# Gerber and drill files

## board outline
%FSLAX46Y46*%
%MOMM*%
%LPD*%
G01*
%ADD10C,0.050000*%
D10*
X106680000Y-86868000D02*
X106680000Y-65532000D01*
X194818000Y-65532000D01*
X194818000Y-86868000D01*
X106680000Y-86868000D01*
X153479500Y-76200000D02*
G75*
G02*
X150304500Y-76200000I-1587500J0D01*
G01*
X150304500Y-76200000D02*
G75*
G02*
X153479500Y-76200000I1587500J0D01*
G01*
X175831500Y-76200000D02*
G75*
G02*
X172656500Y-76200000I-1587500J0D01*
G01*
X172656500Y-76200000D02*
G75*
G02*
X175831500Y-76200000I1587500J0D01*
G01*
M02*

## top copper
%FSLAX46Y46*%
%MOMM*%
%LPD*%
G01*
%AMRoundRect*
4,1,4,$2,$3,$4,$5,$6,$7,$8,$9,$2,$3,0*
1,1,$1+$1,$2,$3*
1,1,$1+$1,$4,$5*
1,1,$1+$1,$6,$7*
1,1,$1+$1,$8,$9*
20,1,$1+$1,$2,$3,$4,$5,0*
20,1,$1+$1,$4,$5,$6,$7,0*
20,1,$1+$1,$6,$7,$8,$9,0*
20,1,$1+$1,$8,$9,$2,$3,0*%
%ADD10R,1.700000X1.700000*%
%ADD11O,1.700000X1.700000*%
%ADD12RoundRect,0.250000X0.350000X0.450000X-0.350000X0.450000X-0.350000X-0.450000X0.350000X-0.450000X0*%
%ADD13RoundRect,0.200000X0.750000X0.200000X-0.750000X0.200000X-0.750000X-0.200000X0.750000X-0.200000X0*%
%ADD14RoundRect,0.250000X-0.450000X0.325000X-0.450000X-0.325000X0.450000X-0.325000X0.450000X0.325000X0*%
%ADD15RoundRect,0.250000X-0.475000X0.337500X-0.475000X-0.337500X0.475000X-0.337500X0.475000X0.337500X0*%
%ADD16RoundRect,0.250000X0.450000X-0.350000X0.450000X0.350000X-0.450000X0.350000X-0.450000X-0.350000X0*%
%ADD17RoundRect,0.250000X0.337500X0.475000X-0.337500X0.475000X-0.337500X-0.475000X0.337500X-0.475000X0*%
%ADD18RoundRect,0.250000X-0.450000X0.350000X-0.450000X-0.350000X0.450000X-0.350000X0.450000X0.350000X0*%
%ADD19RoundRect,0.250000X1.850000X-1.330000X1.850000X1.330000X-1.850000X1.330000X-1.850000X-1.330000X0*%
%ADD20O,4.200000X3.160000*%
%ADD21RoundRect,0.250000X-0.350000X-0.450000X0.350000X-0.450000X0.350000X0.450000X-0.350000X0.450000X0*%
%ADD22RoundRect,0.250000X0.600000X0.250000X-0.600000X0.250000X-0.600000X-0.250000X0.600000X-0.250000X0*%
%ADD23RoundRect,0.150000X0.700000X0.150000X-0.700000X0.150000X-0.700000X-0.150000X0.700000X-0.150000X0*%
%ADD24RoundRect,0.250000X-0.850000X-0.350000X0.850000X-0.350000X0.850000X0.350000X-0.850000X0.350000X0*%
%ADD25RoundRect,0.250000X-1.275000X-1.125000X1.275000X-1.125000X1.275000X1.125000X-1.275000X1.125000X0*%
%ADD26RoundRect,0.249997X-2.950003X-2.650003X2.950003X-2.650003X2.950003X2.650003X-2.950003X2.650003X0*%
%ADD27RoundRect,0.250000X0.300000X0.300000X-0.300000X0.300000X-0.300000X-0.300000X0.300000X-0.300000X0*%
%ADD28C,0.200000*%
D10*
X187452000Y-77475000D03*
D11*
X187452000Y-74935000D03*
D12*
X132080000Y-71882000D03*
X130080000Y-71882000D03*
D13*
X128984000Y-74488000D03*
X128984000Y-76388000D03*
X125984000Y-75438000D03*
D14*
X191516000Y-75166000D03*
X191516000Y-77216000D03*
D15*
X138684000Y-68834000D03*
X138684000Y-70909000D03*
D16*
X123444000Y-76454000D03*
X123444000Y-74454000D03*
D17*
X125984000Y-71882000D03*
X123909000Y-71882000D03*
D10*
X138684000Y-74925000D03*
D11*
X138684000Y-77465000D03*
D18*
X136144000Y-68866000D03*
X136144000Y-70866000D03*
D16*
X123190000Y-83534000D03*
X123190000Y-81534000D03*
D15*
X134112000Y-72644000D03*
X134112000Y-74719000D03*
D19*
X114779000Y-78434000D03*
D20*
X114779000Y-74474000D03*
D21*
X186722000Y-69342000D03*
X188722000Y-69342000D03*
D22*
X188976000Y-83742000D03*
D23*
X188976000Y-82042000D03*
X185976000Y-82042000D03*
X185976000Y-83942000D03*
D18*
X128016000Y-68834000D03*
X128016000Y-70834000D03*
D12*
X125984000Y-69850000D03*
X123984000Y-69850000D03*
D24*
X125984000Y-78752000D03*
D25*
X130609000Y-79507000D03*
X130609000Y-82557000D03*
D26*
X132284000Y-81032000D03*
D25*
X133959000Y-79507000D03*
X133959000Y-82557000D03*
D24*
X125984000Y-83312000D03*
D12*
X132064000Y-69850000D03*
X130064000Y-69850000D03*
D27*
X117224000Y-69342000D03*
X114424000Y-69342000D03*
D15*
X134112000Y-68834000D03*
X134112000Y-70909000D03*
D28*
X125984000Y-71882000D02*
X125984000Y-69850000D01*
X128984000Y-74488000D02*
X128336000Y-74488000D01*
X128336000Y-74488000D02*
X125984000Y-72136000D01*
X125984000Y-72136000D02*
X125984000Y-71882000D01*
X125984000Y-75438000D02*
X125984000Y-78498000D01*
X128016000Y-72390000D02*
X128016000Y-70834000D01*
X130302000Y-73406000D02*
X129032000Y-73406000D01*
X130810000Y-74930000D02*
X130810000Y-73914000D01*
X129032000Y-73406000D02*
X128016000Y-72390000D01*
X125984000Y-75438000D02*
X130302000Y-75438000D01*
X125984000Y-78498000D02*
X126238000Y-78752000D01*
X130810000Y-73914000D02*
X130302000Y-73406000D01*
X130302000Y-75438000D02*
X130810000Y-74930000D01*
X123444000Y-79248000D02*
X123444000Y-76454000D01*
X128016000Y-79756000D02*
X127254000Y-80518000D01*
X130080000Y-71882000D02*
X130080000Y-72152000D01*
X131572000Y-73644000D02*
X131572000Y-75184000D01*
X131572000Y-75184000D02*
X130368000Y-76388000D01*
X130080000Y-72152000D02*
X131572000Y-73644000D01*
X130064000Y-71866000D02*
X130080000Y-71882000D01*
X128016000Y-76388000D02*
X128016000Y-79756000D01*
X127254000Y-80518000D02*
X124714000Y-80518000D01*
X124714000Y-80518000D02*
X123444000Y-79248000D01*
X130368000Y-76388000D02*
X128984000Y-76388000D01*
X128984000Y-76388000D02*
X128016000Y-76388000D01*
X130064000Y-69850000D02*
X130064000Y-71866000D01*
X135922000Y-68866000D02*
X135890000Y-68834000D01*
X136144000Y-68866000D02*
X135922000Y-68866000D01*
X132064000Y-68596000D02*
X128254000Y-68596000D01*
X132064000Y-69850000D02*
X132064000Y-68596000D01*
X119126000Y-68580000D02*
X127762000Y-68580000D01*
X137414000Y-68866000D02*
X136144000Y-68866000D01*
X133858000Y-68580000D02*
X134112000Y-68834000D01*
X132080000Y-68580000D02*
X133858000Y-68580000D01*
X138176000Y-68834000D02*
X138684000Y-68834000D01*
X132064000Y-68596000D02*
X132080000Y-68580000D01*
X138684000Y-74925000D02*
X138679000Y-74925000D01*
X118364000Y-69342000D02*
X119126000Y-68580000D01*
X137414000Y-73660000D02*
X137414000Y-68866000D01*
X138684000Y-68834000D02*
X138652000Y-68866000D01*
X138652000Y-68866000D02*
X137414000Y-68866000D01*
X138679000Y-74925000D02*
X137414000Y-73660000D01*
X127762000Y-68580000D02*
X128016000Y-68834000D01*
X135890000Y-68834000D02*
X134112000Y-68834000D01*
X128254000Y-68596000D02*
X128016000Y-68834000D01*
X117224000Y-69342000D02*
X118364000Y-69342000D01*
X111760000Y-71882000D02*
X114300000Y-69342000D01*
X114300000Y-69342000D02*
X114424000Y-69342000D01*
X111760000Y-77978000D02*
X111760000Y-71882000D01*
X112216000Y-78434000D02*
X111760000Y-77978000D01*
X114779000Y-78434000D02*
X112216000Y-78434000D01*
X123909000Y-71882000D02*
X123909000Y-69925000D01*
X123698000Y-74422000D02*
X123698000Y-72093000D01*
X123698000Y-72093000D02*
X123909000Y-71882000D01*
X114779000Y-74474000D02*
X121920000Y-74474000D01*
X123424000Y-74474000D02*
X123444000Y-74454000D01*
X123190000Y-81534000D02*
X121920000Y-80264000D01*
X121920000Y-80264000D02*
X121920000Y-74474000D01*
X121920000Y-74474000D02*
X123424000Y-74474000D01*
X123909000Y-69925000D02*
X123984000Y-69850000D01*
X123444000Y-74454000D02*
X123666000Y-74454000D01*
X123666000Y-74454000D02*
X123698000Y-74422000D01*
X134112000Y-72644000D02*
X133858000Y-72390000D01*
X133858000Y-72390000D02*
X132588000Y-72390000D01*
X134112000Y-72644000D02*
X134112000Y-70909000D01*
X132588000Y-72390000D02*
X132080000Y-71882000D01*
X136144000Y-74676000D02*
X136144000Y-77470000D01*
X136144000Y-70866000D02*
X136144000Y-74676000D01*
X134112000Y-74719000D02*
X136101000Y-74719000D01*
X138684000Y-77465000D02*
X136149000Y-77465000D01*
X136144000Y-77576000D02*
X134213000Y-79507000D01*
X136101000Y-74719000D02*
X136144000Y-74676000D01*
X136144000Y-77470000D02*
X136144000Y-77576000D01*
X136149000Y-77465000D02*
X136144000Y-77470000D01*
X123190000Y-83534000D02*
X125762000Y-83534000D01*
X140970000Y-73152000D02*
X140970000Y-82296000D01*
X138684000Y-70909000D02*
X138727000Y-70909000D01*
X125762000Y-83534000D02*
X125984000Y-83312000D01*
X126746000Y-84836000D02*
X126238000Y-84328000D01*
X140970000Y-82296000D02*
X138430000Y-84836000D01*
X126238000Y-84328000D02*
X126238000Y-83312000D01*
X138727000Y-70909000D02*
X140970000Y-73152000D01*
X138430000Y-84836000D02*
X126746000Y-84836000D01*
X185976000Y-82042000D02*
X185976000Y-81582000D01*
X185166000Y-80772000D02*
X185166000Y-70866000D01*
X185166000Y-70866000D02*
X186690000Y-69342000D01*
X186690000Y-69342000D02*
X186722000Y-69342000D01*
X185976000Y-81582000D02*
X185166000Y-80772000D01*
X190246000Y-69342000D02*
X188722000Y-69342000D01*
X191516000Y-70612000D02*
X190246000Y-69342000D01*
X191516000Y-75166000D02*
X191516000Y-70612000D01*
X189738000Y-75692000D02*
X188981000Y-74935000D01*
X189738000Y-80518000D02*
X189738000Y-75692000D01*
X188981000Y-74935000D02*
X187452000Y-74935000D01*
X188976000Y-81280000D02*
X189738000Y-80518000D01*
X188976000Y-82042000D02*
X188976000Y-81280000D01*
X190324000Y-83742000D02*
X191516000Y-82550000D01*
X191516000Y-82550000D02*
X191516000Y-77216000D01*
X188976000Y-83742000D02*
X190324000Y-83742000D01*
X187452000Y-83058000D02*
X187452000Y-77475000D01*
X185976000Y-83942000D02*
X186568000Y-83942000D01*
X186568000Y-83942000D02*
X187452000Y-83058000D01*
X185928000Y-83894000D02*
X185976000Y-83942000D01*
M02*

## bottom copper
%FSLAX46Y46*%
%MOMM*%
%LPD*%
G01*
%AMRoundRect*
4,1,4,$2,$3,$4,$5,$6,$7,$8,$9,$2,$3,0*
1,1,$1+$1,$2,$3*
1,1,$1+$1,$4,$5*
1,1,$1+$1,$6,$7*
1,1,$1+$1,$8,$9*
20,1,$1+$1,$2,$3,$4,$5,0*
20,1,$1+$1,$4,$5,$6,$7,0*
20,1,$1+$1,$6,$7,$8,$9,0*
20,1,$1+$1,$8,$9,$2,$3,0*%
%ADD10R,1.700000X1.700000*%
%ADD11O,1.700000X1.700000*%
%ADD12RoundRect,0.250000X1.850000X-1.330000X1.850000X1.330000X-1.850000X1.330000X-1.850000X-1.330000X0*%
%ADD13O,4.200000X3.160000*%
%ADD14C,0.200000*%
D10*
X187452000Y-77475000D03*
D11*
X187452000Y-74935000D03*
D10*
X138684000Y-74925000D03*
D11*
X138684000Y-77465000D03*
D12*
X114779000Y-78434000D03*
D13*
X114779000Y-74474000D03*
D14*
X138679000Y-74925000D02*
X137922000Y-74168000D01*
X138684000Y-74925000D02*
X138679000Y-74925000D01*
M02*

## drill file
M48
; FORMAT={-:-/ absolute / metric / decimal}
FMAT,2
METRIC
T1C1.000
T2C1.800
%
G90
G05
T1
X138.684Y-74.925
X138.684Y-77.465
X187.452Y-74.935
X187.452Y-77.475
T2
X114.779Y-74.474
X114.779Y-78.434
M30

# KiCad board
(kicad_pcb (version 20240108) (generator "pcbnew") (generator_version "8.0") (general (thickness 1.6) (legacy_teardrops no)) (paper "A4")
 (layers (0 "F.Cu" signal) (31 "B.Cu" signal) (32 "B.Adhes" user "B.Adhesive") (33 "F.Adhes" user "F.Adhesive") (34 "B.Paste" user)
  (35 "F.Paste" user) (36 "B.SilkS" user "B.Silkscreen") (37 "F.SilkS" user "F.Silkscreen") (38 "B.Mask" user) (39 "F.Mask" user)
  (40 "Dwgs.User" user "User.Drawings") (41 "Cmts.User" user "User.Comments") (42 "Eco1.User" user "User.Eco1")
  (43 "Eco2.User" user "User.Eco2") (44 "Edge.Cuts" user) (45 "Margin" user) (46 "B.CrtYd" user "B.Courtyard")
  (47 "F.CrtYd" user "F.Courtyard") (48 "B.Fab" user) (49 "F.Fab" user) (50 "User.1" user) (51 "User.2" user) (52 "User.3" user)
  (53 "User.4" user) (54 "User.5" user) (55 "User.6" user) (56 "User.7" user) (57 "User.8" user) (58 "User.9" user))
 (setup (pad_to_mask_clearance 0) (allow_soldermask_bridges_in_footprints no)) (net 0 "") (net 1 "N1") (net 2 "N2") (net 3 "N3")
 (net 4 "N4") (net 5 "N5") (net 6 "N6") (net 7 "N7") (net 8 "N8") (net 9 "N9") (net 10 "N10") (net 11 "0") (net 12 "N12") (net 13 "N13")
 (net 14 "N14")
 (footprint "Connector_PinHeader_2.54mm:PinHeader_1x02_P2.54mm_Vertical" (layer "F.Cu") (at 187.452 77.475 180)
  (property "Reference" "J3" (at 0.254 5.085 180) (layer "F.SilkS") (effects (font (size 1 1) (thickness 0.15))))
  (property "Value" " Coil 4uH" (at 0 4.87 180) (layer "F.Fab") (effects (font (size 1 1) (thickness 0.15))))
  (pad "1" thru_hole rect (at 0 0 180) (size 1.7 1.7) (drill 1) (layers "*.Cu" "*.Mask") (remove_unused_layers no) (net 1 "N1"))
  (pad "2" thru_hole oval (at 0 2.54 180) (size 1.7 1.7) (drill 1) (layers "*.Cu" "*.Mask") (remove_unused_layers no) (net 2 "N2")))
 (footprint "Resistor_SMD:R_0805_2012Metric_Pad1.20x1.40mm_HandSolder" (layer "F.Cu") (at 131.08 71.882 180)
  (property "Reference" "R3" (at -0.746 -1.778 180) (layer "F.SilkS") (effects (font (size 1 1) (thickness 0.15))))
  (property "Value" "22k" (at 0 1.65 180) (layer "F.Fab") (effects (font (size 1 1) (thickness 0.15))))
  (pad "1" smd roundrect (at -1 0 180) (size 1.2 1.4) (layers "F.Cu" "F.Paste" "F.Mask") (roundrect_rratio 0.208333) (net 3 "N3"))
  (pad "2" smd roundrect (at 1 0 180) (size 1.2 1.4) (layers "F.Cu" "F.Paste" "F.Mask") (roundrect_rratio 0.208333) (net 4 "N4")))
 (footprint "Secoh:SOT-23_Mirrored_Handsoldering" (layer "F.Cu") (at 127.484 75.438 180)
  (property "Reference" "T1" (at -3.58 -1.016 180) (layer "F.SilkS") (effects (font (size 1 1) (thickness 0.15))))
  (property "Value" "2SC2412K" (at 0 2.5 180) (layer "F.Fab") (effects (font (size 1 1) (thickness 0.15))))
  (pad "1" smd roundrect (at -1.5 0.95 180) (size 1.9 0.8) (layers "F.Cu" "F.Paste" "F.Mask") (roundrect_rratio 0.25) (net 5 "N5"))
  (pad "2" smd roundrect (at -1.5 -0.95 180) (size 1.9 0.8) (layers "F.Cu" "F.Paste" "F.Mask") (roundrect_rratio 0.25) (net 4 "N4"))
  (pad "3" smd roundrect (at 1.5 0 180) (size 1.9 0.8) (layers "F.Cu" "F.Paste" "F.Mask") (roundrect_rratio 0.25) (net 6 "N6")))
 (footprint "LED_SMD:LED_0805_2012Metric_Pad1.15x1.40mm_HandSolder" (layer "F.Cu") (at 191.516 76.191 -90)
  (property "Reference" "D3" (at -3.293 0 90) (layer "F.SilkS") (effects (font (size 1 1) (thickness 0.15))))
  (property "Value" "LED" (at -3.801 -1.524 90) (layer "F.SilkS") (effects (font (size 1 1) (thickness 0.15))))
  (pad "1" smd roundrect (at -1.025 0 270) (size 1.15 1.4) (layers "F.Cu" "F.Paste" "F.Mask") (roundrect_rratio 0.217391) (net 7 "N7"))
  (pad "2" smd roundrect (at 1.025 0 270) (size 1.15 1.4) (layers "F.Cu" "F.Paste" "F.Mask") (roundrect_rratio 0.217391) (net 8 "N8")))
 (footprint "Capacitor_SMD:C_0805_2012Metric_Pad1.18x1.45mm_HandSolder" (layer "F.Cu") (at 138.684 69.8715 -90)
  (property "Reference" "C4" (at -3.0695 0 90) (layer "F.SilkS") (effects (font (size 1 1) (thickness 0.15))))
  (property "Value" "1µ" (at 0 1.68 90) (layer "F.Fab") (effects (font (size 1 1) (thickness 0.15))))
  (pad "1" smd roundrect (at -1.0375 0 270) (size 1.175 1.45) (layers "F.Cu" "F.Paste" "F.Mask") (roundrect_rratio 0.212766) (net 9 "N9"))
  (pad "2" smd roundrect (at 1.0375 0 270) (size 1.175 1.45) (layers "F.Cu" "F.Paste" "F.Mask") (roundrect_rratio 0.212766) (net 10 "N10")))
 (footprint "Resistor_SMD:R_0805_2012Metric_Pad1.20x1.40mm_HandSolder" (layer "F.Cu") (at 123.444 75.454 90)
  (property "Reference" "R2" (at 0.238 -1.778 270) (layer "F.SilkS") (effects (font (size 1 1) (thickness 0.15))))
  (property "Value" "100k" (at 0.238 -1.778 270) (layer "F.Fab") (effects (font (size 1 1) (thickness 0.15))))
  (pad "1" smd roundrect (at -1 0 90) (size 1.2 1.4) (layers "F.Cu" "F.Paste" "F.Mask") (roundrect_rratio 0.208333) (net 4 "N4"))
  (pad "2" smd roundrect (at 1 0 90) (size 1.2 1.4) (layers "F.Cu" "F.Paste" "F.Mask") (roundrect_rratio 0.208333) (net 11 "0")))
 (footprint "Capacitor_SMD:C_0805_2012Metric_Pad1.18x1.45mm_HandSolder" (layer "F.Cu") (at 124.9465 71.882 180)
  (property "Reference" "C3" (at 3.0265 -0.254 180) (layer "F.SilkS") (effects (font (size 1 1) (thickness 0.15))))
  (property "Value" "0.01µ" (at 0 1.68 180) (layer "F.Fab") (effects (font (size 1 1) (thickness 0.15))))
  (pad "1" smd roundrect (at -1.0375 0 180) (size 1.175 1.45) (layers "F.Cu" "F.Paste" "F.Mask") (roundrect_rratio 0.212766) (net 5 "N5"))
  (pad "2" smd roundrect (at 1.0375 0 180) (size 1.175 1.45) (layers "F.Cu" "F.Paste" "F.Mask") (roundrect_rratio 0.212766) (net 11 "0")))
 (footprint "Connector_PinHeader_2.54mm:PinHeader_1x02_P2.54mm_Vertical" (layer "F.Cu") (at 138.684 74.925)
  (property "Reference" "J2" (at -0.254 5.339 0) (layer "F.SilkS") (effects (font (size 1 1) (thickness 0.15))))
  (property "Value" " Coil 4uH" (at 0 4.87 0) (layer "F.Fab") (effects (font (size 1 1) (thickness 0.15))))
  (pad "1" thru_hole rect (at 0 0) (size 1.7 1.7) (drill 1) (layers "*.Cu" "*.Mask") (remove_unused_layers no) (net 9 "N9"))
  (pad "2" thru_hole oval (at 0 2.54) (size 1.7 1.7) (drill 1) (layers "*.Cu" "*.Mask") (remove_unused_layers no) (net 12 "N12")))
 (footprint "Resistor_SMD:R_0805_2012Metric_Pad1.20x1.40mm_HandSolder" (layer "F.Cu") (at 136.144 69.866 -90)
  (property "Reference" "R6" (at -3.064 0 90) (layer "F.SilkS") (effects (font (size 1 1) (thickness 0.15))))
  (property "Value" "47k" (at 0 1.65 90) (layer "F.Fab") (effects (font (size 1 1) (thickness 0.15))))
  (pad "1" smd roundrect (at -1 0 270) (size 1.2 1.4) (layers "F.Cu" "F.Paste" "F.Mask") (roundrect_rratio 0.208333) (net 9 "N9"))
  (pad "2" smd roundrect (at 1 0 270) (size 1.2 1.4) (layers "F.Cu" "F.Paste" "F.Mask") (roundrect_rratio 0.208333) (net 12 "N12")))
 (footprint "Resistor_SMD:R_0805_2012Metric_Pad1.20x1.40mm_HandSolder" (layer "F.Cu") (at 123.19 82.534 90)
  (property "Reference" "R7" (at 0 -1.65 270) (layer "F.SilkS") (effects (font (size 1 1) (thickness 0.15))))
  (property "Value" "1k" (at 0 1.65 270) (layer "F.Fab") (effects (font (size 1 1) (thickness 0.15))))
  (pad "1" smd roundrect (at -1 0 90) (size 1.2 1.4) (layers "F.Cu" "F.Paste" "F.Mask") (roundrect_rratio 0.208333) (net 10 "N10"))
  (pad "2" smd roundrect (at 1 0 90) (size 1.2 1.4) (layers "F.Cu" "F.Paste" "F.Mask") (roundrect_rratio 0.208333) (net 11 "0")))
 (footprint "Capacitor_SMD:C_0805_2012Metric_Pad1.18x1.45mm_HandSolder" (layer "F.Cu") (at 134.112 73.6815 -90)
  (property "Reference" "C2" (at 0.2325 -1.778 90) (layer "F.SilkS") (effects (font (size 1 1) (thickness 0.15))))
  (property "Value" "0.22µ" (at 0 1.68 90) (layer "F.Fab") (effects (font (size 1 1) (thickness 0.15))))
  (pad "1" smd roundrect (at -1.0375 0 270) (size 1.175 1.45) (layers "F.Cu" "F.Paste" "F.Mask") (roundrect_rratio 0.212766) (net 3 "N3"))
  (pad "2" smd roundrect (at 1.0375 0 270) (size 1.175 1.45) (layers "F.Cu" "F.Paste" "F.Mask") (roundrect_rratio 0.212766) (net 12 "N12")))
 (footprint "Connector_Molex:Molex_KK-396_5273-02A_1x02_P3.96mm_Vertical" (layer "F.Cu") (at 114.779 78.434 90)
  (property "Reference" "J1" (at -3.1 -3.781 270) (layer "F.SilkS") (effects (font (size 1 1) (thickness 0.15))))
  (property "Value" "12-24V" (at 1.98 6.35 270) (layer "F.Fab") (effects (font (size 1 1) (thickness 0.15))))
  (pad "1" thru_hole roundrect (at 0 0 90) (size 3.16 4.2) (drill 1.8) (layers "*.Cu" "*.Mask") (remove_unused_layers no)
   (roundrect_rratio 0.079114) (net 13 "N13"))
  (pad "2" thru_hole oval (at 3.96 0 90) (size 3.16 4.2) (drill 1.8) (layers "*.Cu" "*.Mask") (remove_unused_layers no) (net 11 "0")))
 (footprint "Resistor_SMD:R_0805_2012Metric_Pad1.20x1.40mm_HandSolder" (layer "F.Cu") (at 187.722 69.342)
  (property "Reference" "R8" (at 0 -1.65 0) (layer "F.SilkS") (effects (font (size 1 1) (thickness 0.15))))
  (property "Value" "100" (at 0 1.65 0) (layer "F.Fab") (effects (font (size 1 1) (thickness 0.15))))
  (pad "1" smd roundrect (at -1 0) (size 1.2 1.4) (layers "F.Cu" "F.Paste" "F.Mask") (roundrect_rratio 0.208333) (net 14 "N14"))
  (pad "2" smd roundrect (at 1 0) (size 1.2 1.4) (layers "F.Cu" "F.Paste" "F.Mask") (roundrect_rratio 0.208333) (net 7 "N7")))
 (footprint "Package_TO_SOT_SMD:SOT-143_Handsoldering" (layer "F.Cu") (at 187.476 82.992 180)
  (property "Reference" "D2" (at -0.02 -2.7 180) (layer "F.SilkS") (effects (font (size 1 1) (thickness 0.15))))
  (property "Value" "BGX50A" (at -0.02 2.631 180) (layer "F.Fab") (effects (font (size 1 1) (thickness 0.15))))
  (pad "1" smd roundrect (at -1.5 -0.75 180) (size 1.7 1) (layers "F.Cu" "F.Paste" "F.Mask") (roundrect_rratio 0.25) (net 8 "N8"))
  (pad "2" smd roundrect (at -1.5 0.95 180) (size 1.7 0.6) (layers "F.Cu" "F.Paste" "F.Mask") (roundrect_rratio 0.25) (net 2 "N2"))
  (pad "3" smd roundrect (at 1.5 0.95 180) (size 1.7 0.6) (layers "F.Cu" "F.Paste" "F.Mask") (roundrect_rratio 0.25) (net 14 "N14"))
  (pad "4" smd roundrect (at 1.5 -0.95 180) (size 1.7 0.6) (layers "F.Cu" "F.Paste" "F.Mask") (roundrect_rratio 0.25) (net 1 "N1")))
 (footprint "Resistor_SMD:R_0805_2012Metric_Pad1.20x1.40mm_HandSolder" (layer "F.Cu") (at 128.016 69.834 -90)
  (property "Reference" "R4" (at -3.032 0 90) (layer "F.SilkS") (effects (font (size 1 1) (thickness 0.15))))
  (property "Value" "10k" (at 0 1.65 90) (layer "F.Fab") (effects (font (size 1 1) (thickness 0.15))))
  (pad "1" smd roundrect (at -1 0 270) (size 1.2 1.4) (layers "F.Cu" "F.Paste" "F.Mask") (roundrect_rratio 0.208333) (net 9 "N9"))
  (pad "2" smd roundrect (at 1 0 270) (size 1.2 1.4) (layers "F.Cu" "F.Paste" "F.Mask") (roundrect_rratio 0.208333) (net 6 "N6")))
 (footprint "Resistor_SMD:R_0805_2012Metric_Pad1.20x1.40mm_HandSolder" (layer "F.Cu") (at 124.984 69.85 180)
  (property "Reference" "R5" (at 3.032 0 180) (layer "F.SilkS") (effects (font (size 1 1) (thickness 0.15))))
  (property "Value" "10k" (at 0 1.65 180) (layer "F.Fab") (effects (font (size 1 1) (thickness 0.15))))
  (pad "1" smd roundrect (at -1 0 180) (size 1.2 1.4) (layers "F.Cu" "F.Paste" "F.Mask") (roundrect_rratio 0.208333) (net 5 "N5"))
  (pad "2" smd roundrect (at 1 0 180) (size 1.2 1.4) (layers "F.Cu" "F.Paste" "F.Mask") (roundrect_rratio 0.208333) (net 11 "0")))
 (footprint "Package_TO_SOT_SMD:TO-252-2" (layer "F.Cu") (at 131.024 81.032)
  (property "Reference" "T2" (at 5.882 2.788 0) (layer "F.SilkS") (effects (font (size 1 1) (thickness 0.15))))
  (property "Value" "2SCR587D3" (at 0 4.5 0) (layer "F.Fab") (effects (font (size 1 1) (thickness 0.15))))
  (pad "1" smd roundrect (at -5.04 -2.28) (size 2.2 1.2) (layers "F.Cu" "F.Paste" "F.Mask") (roundrect_rratio 0.208333) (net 6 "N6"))
  (pad "2" smd roundrect (at -0.415 -1.525) (size 3.05 2.75) (layers "F.Cu" "F.Paste") (roundrect_rratio 0.090909) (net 12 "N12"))
  (pad "2" smd roundrect (at -0.415 1.525) (size 3.05 2.75) (layers "F.Cu" "F.Paste") (roundrect_rratio 0.090909) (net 12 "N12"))
  (pad "2" smd roundrect (at 1.26 0) (size 6.4 5.8) (layers "F.Cu" "F.Mask") (roundrect_rratio 0.043103) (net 12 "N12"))
  (pad "2" smd roundrect (at 2.935 -1.525) (size 3.05 2.75) (layers "F.Cu" "F.Paste") (roundrect_rratio 0.090909) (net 12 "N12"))
  (pad "2" smd roundrect (at 2.935 1.525) (size 3.05 2.75) (layers "F.Cu" "F.Paste") (roundrect_rratio 0.090909) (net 12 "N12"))
  (pad "3" smd roundrect (at -5.04 2.28) (size 2.2 1.2) (layers "F.Cu" "F.Paste" "F.Mask") (roundrect_rratio 0.208333) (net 10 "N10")))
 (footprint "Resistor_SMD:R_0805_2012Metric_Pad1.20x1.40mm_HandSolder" (layer "F.Cu") (at 131.064 69.85 180)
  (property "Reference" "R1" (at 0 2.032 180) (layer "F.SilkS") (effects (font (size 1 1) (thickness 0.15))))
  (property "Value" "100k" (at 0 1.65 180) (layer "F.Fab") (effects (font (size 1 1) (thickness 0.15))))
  (pad "1" smd roundrect (at -1 0 180) (size 1.2 1.4) (layers "F.Cu" "F.Paste" "F.Mask") (roundrect_rratio 0.208333) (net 9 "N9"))
  (pad "2" smd roundrect (at 1 0 180) (size 1.2 1.4) (layers "F.Cu" "F.Paste" "F.Mask") (roundrect_rratio 0.208333) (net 4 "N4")))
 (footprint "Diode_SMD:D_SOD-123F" (layer "F.Cu") (at 115.824 69.342 180)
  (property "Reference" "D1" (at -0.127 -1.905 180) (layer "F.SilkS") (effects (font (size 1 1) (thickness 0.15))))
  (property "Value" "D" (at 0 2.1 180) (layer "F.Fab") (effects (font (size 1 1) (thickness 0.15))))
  (pad "1" smd roundrect (at -1.4 0 180) (size 1.1 1.1) (layers "F.Cu" "F.Paste" "F.Mask") (roundrect_rratio 0.2272727273) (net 9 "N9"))
  (pad "2" smd roundrect (at 1.4 0 180) (size 1.1 1.1) (layers "F.Cu" "F.Paste" "F.Mask") (roundrect_rratio 0.2272727273) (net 13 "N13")))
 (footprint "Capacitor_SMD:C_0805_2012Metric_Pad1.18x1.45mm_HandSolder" (layer "F.Cu") (at 134.112 69.8715 -90)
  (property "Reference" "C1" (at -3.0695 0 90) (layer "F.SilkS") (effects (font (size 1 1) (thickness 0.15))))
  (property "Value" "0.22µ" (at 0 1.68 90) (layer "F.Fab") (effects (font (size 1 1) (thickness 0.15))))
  (pad "1" smd roundrect (at -1.0375 0 270) (size 1.175 1.45) (layers "F.Cu" "F.Paste" "F.Mask") (roundrect_rratio 0.212766) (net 9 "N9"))
  (pad "2" smd roundrect (at 1.0375 0 270) (size 1.175 1.45) (layers "F.Cu" "F.Paste" "F.Mask") (roundrect_rratio 0.212766) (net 3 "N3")))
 (gr_poly
  (pts (xy 106.68 86.868) (xy 106.68 65.532) (xy 194.818 65.532) (xy 194.818 86.868)) (stroke (width 0.05) (type solid)) (fill none)
  (layer "Edge.Cuts"))
 (gr_circle (center 151.892 76.2) (end 153.4795 76.2) (stroke (width 0.05) (type default)) (fill none) (layer "Edge.Cuts"))
 (gr_circle (center 174.244 76.2) (end 175.8315 76.2) (stroke (width 0.05) (type default)) (fill none) (layer "Edge.Cuts"))
 (segment (start 125.984 71.882) (end 125.984 69.85) (width 0.2) (layer "F.Cu") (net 5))
 (segment (start 128.984 74.488) (end 128.336 74.488) (width 0.2) (layer "F.Cu") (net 5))
 (segment (start 128.336 74.488) (end 125.984 72.136) (width 0.2) (layer "F.Cu") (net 5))
 (segment (start 125.984 72.136) (end 125.984 71.882) (width 0.2) (layer "F.Cu") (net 5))
 (segment (start 125.984 75.438) (end 125.984 78.498) (width 0.2) (layer "F.Cu") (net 6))
 (segment (start 128.016 72.39) (end 128.016 70.834) (width 0.2) (layer "F.Cu") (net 6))
 (segment (start 130.302 73.406) (end 129.032 73.406) (width 0.2) (layer "F.Cu") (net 6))
 (segment (start 130.81 74.93) (end 130.81 73.914) (width 0.2) (layer "F.Cu") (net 6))
 (segment (start 129.032 73.406) (end 128.016 72.39) (width 0.2) (layer "F.Cu") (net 6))
 (segment (start 125.984 75.438) (end 130.302 75.438) (width 0.2) (layer "F.Cu") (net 6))
 (segment (start 125.984 78.498) (end 126.238 78.752) (width 0.2) (layer "F.Cu") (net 6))
 (segment (start 130.81 73.914) (end 130.302 73.406) (width 0.2) (layer "F.Cu") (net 6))
 (segment (start 130.302 75.438) (end 130.81 74.93) (width 0.2) (layer "F.Cu") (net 6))
 (segment (start 123.444 79.248) (end 123.444 76.454) (width 0.2) (layer "F.Cu") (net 4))
 (segment (start 128.016 79.756) (end 127.254 80.518) (width 0.2) (layer "F.Cu") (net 4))
 (segment (start 130.08 71.882) (end 130.08 72.152) (width 0.2) (layer "F.Cu") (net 4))
 (segment (start 131.572 73.644) (end 131.572 75.184) (width 0.2) (layer "F.Cu") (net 4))
 (segment (start 131.572 75.184) (end 130.368 76.388) (width 0.2) (layer "F.Cu") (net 4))
 (segment (start 130.08 72.152) (end 131.572 73.644) (width 0.2) (layer "F.Cu") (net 4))
 (segment (start 130.064 71.866) (end 130.08 71.882) (width 0.2) (layer "F.Cu") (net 4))
 (segment (start 128.016 76.388) (end 128.016 79.756) (width 0.2) (layer "F.Cu") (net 4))
 (segment (start 127.254 80.518) (end 124.714 80.518) (width 0.2) (layer "F.Cu") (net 4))
 (segment (start 124.714 80.518) (end 123.444 79.248) (width 0.2) (layer "F.Cu") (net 4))
 (segment (start 130.368 76.388) (end 128.984 76.388) (width 0.2) (layer "F.Cu") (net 4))
 (segment (start 128.984 76.388) (end 128.016 76.388) (width 0.2) (layer "F.Cu") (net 4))
 (segment (start 130.064 69.85) (end 130.064 71.866) (width 0.2) (layer "F.Cu") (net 4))
 (segment (start 135.922 68.866) (end 135.89 68.834) (width 0.2) (layer "F.Cu") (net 9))
 (segment (start 136.144 68.866) (end 135.922 68.866) (width 0.2) (layer "F.Cu") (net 9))
 (segment (start 132.064 68.596) (end 128.254 68.596) (width 0.2) (layer "F.Cu") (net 9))
 (segment (start 132.064 69.85) (end 132.064 68.596) (width 0.2) (layer "F.Cu") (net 9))
 (segment (start 119.126 68.58) (end 127.762 68.58) (width 0.2) (layer "F.Cu") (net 9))
 (segment (start 137.414 68.866) (end 136.144 68.866) (width 0.2) (layer "F.Cu") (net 9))
 (segment (start 133.858 68.58) (end 134.112 68.834) (width 0.2) (layer "F.Cu") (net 9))
 (segment (start 132.08 68.58) (end 133.858 68.58) (width 0.2) (layer "F.Cu") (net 9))
 (segment (start 138.176 68.834) (end 138.684 68.834) (width 0.2) (layer "F.Cu") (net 9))
 (segment (start 132.064 68.596) (end 132.08 68.58) (width 0.2) (layer "F.Cu") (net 9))
 (segment (start 138.684 74.925) (end 138.679 74.925) (width 0.2) (layer "F.Cu") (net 9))
 (segment (start 118.364 69.342) (end 119.126 68.58) (width 0.2) (layer "F.Cu") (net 9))
 (segment (start 137.414 73.66) (end 137.414 68.866) (width 0.2) (layer "F.Cu") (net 9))
 (segment (start 138.684 68.834) (end 138.652 68.866) (width 0.2) (layer "F.Cu") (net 9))
 (segment (start 138.652 68.866) (end 137.414 68.866) (width 0.2) (layer "F.Cu") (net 9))
 (segment (start 138.679 74.925) (end 137.414 73.66) (width 0.2) (layer "F.Cu") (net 9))
 (segment (start 127.762 68.58) (end 128.016 68.834) (width 0.2) (layer "F.Cu") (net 9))
 (segment (start 135.89 68.834) (end 134.112 68.834) (width 0.2) (layer "F.Cu") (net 9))
 (segment (start 128.254 68.596) (end 128.016 68.834) (width 0.2) (layer "F.Cu") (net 9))
 (segment (start 117.224 69.342) (end 118.364 69.342) (width 0.2) (layer "F.Cu") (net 9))
 (segment (start 138.679 74.925) (end 137.922 74.168) (width 0.2) (layer "B.Cu") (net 9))
 (segment (start 138.684 74.925) (end 138.679 74.925) (width 0.2) (layer "B.Cu") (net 9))
 (segment (start 111.76 71.882) (end 114.3 69.342) (width 0.2) (layer "F.Cu") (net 13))
 (segment (start 114.3 69.342) (end 114.424 69.342) (width 0.2) (layer "F.Cu") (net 13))
 (segment (start 111.76 77.978) (end 111.76 71.882) (width 0.2) (layer "F.Cu") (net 13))
 (segment (start 112.216 78.434) (end 111.76 77.978) (width 0.2) (layer "F.Cu") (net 13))
 (segment (start 114.779 78.434) (end 112.216 78.434) (width 0.2) (layer "F.Cu") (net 13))
 (segment (start 123.909 71.882) (end 123.909 69.925) (width 0.2) (layer "F.Cu") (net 11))
 (segment (start 123.698 74.422) (end 123.698 72.093) (width 0.2) (layer "F.Cu") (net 11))
 (segment (start 123.698 72.093) (end 123.909 71.882) (width 0.2) (layer "F.Cu") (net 11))
 (segment (start 114.779 74.474) (end 121.92 74.474) (width 0.2) (layer "F.Cu") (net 11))
 (segment (start 123.424 74.474) (end 123.444 74.454) (width 0.2) (layer "F.Cu") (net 11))
 (segment (start 123.19 81.534) (end 121.92 80.264) (width 0.2) (layer "F.Cu") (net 11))
 (segment (start 121.92 80.264) (end 121.92 74.474) (width 0.2) (layer "F.Cu") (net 11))
 (segment (start 121.92 74.474) (end 123.424 74.474) (width 0.2) (layer "F.Cu") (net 11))
 (segment (start 123.909 69.925) (end 123.984 69.85) (width 0.2) (layer "F.Cu") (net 11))
 (segment (start 123.444 74.454) (end 123.666 74.454) (width 0.2) (layer "F.Cu") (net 11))
 (segment (start 123.666 74.454) (end 123.698 74.422) (width 0.2) (layer "F.Cu") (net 11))
 (segment (start 134.112 72.644) (end 133.858 72.39) (width 0.2) (layer "F.Cu") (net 3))
 (segment (start 133.858 72.39) (end 132.588 72.39) (width 0.2) (layer "F.Cu") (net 3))
 (segment (start 134.112 72.644) (end 134.112 70.909) (width 0.2) (layer "F.Cu") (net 3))
 (segment (start 132.588 72.39) (end 132.08 71.882) (width 0.2) (layer "F.Cu") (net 3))
 (segment (start 136.144 74.676) (end 136.144 77.47) (width 0.2) (layer "F.Cu") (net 12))
 (segment (start 136.144 70.866) (end 136.144 74.676) (width 0.2) (layer "F.Cu") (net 12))
 (segment (start 134.112 74.719) (end 136.101 74.719) (width 0.2) (layer "F.Cu") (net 12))
 (segment (start 138.684 77.465) (end 136.149 77.465) (width 0.2) (layer "F.Cu") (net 12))
 (segment (start 136.144 77.576) (end 134.213 79.507) (width 0.2) (layer "F.Cu") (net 12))
 (segment (start 136.101 74.719) (end 136.144 74.676) (width 0.2) (layer "F.Cu") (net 12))
 (segment (start 136.144 77.47) (end 136.144 77.576) (width 0.2) (layer "F.Cu") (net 12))
 (segment (start 136.149 77.465) (end 136.144 77.47) (width 0.2) (layer "F.Cu") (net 12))
 (segment (start 123.19 83.534) (end 125.762 83.534) (width 0.2) (layer "F.Cu") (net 10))
 (segment (start 140.97 73.152) (end 140.97 82.296) (width 0.2) (layer "F.Cu") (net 10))
 (segment (start 138.684 70.909) (end 138.727 70.909) (width 0.2) (layer "F.Cu") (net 10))
 (segment (start 125.762 83.534) (end 125.984 83.312) (width 0.2) (layer "F.Cu") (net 10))
 (segment (start 126.746 84.836) (end 126.238 84.328) (width 0.2) (layer "F.Cu") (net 10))
 (segment (start 140.97 82.296) (end 138.43 84.836) (width 0.2) (layer "F.Cu") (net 10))
 (segment (start 126.238 84.328) (end 126.238 83.312) (width 0.2) (layer "F.Cu") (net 10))
 (segment (start 138.727 70.909) (end 140.97 73.152) (width 0.2) (layer "F.Cu") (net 10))
 (segment (start 138.43 84.836) (end 126.746 84.836) (width 0.2) (layer "F.Cu") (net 10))
 (segment (start 185.976 82.042) (end 185.976 81.582) (width 0.2) (layer "F.Cu") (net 14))
 (segment (start 185.166 80.772) (end 185.166 70.866) (width 0.2) (layer "F.Cu") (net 14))
 (segment (start 185.166 70.866) (end 186.69 69.342) (width 0.2) (layer "F.Cu") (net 14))
 (segment (start 186.69 69.342) (end 186.722 69.342) (width 0.2) (layer "F.Cu") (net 14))
 (segment (start 185.976 81.582) (end 185.166 80.772) (width 0.2) (layer "F.Cu") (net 14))
 (segment (start 190.246 69.342) (end 188.722 69.342) (width 0.2) (layer "F.Cu") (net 7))
 (segment (start 191.516 70.612) (end 190.246 69.342) (width 0.2) (layer "F.Cu") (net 7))
 (segment (start 191.516 75.166) (end 191.516 70.612) (width 0.2) (layer "F.Cu") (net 7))
 (segment (start 189.738 75.692) (end 188.981 74.935) (width 0.2) (layer "F.Cu") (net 2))
 (segment (start 189.738 80.518) (end 189.738 75.692) (width 0.2) (layer "F.Cu") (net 2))
 (segment (start 188.981 74.935) (end 187.452 74.935) (width 0.2) (layer "F.Cu") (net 2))
 (segment (start 188.976 81.28) (end 189.738 80.518) (width 0.2) (layer "F.Cu") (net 2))
 (segment (start 188.976 82.042) (end 188.976 81.28) (width 0.2) (layer "F.Cu") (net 2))
 (segment (start 190.324 83.742) (end 191.516 82.55) (width 0.2) (layer "F.Cu") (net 8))
 (segment (start 191.516 82.55) (end 191.516 77.216) (width 0.2) (layer "F.Cu") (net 8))
 (segment (start 188.976 83.742) (end 190.324 83.742) (width 0.2) (layer "F.Cu") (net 8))
 (segment (start 187.452 83.058) (end 187.452 77.475) (width 0.2) (layer "F.Cu") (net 1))
 (segment (start 185.976 83.942) (end 186.568 83.942) (width 0.2) (layer "F.Cu") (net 1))
 (segment (start 186.568 83.942) (end 187.452 83.058) (width 0.2) (layer "F.Cu") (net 1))
 (segment (start 185.928 83.894) (end 185.976 83.942) (width 0.2) (layer "F.Cu") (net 1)))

